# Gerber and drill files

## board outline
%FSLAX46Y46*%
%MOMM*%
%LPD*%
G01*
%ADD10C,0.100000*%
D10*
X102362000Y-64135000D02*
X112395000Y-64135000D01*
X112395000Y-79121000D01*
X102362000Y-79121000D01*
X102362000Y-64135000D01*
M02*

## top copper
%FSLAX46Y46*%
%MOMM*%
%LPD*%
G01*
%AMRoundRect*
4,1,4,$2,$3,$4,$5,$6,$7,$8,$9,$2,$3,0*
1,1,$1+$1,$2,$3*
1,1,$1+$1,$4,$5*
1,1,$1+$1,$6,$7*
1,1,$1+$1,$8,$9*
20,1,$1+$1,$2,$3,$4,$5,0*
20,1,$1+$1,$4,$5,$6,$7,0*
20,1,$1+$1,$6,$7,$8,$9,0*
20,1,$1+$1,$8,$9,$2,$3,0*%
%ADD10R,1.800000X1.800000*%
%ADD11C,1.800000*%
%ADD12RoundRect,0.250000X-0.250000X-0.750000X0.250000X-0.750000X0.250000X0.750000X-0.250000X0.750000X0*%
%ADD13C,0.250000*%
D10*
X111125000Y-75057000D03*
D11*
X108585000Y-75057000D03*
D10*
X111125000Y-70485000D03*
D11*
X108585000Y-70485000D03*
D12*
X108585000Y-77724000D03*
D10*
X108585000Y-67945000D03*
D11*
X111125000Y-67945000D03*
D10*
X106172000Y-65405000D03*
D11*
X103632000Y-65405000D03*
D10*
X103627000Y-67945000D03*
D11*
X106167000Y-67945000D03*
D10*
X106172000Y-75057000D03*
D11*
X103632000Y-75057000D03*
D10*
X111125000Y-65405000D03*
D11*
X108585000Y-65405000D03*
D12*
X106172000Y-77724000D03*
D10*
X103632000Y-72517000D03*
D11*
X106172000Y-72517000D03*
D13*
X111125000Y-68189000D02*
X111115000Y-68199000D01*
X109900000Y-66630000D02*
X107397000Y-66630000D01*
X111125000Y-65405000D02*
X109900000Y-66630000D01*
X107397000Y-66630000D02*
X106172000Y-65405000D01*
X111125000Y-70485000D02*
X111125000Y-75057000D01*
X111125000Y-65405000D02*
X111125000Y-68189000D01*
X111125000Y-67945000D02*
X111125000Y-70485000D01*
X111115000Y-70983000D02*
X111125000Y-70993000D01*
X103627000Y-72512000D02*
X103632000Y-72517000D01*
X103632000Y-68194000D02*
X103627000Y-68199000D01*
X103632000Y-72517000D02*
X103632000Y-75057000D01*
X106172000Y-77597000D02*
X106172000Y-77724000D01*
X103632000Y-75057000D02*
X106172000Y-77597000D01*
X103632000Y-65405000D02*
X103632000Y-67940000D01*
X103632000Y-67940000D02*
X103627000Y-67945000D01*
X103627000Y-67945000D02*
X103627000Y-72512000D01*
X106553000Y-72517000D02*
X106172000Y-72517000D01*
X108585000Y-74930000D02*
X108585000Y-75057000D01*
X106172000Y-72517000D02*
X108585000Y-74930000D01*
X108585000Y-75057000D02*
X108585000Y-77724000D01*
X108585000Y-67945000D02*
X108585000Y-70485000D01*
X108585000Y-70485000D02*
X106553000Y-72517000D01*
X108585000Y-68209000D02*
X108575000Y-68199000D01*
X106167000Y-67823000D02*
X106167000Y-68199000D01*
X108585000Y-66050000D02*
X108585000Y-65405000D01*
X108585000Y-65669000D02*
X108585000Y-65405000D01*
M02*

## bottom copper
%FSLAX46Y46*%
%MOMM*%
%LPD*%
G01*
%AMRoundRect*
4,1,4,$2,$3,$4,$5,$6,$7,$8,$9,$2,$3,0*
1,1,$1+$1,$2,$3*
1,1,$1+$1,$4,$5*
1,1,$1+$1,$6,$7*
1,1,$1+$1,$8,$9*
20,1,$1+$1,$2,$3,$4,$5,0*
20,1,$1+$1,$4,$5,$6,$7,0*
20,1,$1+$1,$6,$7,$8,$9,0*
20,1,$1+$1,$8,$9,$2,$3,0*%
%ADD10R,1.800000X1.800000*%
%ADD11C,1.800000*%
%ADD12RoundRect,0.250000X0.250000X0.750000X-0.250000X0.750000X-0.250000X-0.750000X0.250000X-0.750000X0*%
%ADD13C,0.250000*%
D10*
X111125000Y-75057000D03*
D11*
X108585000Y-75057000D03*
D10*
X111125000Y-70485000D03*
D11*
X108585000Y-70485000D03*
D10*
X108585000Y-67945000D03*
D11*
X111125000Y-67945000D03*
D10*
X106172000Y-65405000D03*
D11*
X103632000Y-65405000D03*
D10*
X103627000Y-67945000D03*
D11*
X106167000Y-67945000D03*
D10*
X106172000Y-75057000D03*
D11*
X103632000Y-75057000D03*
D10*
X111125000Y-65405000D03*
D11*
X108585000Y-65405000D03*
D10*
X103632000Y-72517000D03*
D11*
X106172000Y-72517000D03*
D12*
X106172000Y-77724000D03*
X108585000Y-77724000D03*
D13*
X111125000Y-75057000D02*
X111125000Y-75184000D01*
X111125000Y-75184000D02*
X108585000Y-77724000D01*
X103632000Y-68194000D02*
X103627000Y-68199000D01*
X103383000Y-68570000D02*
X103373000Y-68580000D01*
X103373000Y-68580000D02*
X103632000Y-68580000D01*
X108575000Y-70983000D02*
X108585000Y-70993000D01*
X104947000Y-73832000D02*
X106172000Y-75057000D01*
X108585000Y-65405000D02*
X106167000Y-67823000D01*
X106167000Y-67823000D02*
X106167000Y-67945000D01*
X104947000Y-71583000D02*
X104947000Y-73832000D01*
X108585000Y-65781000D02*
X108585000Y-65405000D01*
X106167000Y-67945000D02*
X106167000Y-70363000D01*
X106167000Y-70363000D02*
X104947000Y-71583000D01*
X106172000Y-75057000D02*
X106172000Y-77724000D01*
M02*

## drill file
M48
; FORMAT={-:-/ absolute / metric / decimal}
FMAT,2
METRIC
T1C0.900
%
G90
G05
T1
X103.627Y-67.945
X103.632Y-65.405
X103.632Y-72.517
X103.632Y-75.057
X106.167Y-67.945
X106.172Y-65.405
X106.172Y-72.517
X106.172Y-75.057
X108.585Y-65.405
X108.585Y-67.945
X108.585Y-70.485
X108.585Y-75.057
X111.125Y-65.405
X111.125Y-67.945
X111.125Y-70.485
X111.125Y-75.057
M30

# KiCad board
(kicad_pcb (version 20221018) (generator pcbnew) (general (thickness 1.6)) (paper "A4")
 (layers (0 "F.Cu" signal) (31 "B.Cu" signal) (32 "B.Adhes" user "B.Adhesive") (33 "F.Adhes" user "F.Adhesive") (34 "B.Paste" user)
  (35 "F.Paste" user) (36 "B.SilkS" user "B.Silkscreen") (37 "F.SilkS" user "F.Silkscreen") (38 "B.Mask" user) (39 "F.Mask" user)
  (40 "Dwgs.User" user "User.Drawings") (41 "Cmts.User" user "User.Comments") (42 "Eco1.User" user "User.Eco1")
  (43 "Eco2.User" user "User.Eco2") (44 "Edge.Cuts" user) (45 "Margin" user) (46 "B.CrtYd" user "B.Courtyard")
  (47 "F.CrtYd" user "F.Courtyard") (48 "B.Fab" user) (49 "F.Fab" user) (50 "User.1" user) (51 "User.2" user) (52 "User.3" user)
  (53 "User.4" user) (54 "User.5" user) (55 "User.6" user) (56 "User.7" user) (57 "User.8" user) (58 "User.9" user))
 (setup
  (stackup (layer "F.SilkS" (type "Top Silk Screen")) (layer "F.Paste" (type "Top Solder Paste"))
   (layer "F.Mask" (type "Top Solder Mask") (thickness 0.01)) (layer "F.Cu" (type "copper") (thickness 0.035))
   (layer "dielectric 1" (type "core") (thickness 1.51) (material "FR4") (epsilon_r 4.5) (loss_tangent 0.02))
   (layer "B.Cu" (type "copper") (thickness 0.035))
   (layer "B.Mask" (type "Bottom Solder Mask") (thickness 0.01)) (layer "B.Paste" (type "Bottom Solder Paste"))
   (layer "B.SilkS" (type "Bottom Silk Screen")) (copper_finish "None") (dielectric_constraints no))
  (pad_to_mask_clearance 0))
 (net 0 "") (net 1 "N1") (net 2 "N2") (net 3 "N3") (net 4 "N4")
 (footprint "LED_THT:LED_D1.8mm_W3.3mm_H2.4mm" (layer "F.Cu") (at 111.125 75.057 180)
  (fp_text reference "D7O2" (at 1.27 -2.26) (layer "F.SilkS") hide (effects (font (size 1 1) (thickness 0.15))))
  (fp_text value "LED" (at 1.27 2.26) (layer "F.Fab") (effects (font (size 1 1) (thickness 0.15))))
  (pad "1" thru_hole rect (at 0 0 180) (size 1.8 1.8) (drill 0.9) (layers "*.Cu" "*.Mask") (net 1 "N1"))
  (pad "2" thru_hole circle (at 2.54 0 180) (size 1.8 1.8) (drill 0.9) (layers "*.Cu" "*.Mask") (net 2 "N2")))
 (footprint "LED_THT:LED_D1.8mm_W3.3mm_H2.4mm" (layer "F.Cu") (at 111.125 70.485 180)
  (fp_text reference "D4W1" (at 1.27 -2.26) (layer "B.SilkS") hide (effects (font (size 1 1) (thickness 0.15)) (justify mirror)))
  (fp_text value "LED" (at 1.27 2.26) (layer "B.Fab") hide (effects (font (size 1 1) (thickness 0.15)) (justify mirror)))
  (pad "1" thru_hole rect (at 0 0 180) (size 1.8 1.8) (drill 0.9) (layers "*.Cu" "*.Mask") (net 1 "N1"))
  (pad "2" thru_hole circle (at 2.54 0 180) (size 1.8 1.8) (drill 0.9) (layers "*.Cu" "*.Mask") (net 2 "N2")))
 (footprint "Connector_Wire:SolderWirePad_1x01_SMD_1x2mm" (layer "F.Cu") (at 108.585 77.724)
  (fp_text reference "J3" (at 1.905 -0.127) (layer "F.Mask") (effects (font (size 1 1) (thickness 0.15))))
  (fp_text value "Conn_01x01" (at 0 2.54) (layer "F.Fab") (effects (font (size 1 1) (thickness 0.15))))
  (pad "1" smd roundrect (at 0 0) (size 1 2) (layers "F.Cu" "F.Paste" "F.Mask") (roundrect_rratio 0.25) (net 2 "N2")))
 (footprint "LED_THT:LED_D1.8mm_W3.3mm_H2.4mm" (layer "F.Cu") (at 108.585 67.945)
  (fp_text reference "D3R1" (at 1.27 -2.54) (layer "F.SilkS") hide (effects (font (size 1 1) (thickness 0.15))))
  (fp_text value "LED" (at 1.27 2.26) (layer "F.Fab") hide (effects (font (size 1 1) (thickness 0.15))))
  (pad "1" thru_hole rect (at 0 0) (size 1.8 1.8) (drill 0.9) (layers "*.Cu" "*.Mask") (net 2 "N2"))
  (pad "2" thru_hole circle (at 2.54 0) (size 1.8 1.8) (drill 0.9) (layers "*.Cu" "*.Mask") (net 1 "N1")))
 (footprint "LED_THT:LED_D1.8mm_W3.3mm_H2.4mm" (layer "F.Cu") (at 106.172 65.405 180)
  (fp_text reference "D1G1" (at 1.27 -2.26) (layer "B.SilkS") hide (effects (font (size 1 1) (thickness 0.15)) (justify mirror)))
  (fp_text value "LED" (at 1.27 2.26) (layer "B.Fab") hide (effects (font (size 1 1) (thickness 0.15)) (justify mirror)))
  (pad "1" thru_hole rect (at 0 0 180) (size 1.8 1.8) (drill 0.9) (layers "*.Cu" "*.Mask") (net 1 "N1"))
  (pad "2" thru_hole circle (at 2.54 0 180) (size 1.8 1.8) (drill 0.9) (layers "*.Cu" "*.Mask") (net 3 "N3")))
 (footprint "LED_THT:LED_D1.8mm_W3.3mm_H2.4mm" (layer "F.Cu") (at 103.627 67.945)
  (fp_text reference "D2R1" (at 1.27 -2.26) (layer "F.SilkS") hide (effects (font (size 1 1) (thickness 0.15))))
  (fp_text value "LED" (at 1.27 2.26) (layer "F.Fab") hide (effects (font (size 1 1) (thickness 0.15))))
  (pad "1" thru_hole rect (at 0 0) (size 1.8 1.8) (drill 0.9) (layers "*.Cu" "*.Mask") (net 3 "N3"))
  (pad "2" thru_hole circle (at 2.54 0) (size 1.8 1.8) (drill 0.9) (layers "*.Cu" "*.Mask") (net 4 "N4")))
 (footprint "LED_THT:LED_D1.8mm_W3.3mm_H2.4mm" (layer "F.Cu") (at 106.172 75.057 180)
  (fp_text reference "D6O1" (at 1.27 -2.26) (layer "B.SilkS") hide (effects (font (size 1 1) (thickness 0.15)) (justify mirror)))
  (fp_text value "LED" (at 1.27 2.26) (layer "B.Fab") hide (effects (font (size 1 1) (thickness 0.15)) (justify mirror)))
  (pad "1" thru_hole rect (at 0 0 180) (size 1.8 1.8) (drill 0.9) (layers "*.Cu" "*.Mask") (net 4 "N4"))
  (pad "2" thru_hole circle (at 2.54 0 180) (size 1.8 1.8) (drill 0.9) (layers "*.Cu" "*.Mask") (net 3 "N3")))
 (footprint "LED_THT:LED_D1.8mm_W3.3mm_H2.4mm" (layer "F.Cu") (at 111.125 65.405 180)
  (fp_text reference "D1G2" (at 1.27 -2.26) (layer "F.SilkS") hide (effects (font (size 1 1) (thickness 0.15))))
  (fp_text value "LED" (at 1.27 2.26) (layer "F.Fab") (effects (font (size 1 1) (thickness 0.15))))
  (pad "1" thru_hole rect (at 0 0 180) (size 1.8 1.8) (drill 0.9) (layers "*.Cu" "*.Mask") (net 1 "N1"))
  (pad "2" thru_hole circle (at 2.54 0 180) (size 1.8 1.8) (drill 0.9) (layers "*.Cu" "*.Mask") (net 4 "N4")))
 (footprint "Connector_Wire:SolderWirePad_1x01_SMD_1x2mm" (layer "F.Cu") (at 106.172 77.724)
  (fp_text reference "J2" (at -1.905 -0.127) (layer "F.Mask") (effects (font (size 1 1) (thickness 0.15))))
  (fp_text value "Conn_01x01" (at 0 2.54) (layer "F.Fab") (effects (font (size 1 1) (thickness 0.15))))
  (pad "1" smd roundrect (at 0 0) (size 1 2) (layers "F.Cu" "F.Paste" "F.Mask") (roundrect_rratio 0.25) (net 3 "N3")))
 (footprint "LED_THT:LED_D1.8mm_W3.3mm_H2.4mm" (layer "F.Cu") (at 103.632 72.517)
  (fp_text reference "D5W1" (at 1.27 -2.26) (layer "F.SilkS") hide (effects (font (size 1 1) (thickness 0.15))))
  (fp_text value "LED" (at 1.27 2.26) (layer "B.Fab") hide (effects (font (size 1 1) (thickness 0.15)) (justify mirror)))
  (pad "1" thru_hole rect (at 0 0) (size 1.8 1.8) (drill 0.9) (layers "*.Cu" "*.Mask") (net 3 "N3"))
  (pad "2" thru_hole circle (at 2.54 0) (size 1.8 1.8) (drill 0.9) (layers "*.Cu" "*.Mask") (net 2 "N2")))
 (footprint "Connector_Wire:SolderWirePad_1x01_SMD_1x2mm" (layer "B.Cu") (at 106.172 77.724 180)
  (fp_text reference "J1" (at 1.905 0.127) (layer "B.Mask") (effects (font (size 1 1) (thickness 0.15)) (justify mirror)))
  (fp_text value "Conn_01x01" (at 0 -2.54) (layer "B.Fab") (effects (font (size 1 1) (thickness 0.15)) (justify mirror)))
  (pad "1" smd roundrect (at 0 0 180) (size 1 2) (layers "B.Cu" "B.Paste" "B.Mask") (roundrect_rratio 0.25) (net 4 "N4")))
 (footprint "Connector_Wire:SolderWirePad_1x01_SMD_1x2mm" (layer "B.Cu") (at 108.585 77.724 180)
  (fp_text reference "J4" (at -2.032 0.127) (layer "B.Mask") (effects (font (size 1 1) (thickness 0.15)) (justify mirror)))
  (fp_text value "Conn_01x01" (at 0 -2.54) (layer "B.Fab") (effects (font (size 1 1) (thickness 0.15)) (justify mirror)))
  (pad "1" smd roundrect (at 0 0 180) (size 1 2) (layers "B.Cu" "B.Paste" "B.Mask") (roundrect_rratio 0.25) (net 1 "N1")))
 (gr_rect (start 102.362 64.135) (end 112.395 79.121) (stroke (width 0.1) (type default)) (fill none) (layer "Edge.Cuts"))
 (segment (start 111.125 68.189) (end 111.115 68.199) (width 0.25) (layer "F.Cu") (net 1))
 (segment (start 109.9 66.63) (end 107.397 66.63) (width 0.25) (layer "F.Cu") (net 1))
 (segment (start 111.125 65.405) (end 109.9 66.63) (width 0.25) (layer "F.Cu") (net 1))
 (segment (start 107.397 66.63) (end 106.172 65.405) (width 0.25) (layer "F.Cu") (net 1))
 (segment (start 111.125 70.485) (end 111.125 75.057) (width 0.25) (layer "F.Cu") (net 1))
 (segment (start 111.125 65.405) (end 111.125 68.189) (width 0.25) (layer "F.Cu") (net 1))
 (segment (start 111.125 67.945) (end 111.125 70.485) (width 0.25) (layer "F.Cu") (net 1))
 (segment (start 111.115 70.983) (end 111.125 70.993) (width 0.25) (layer "F.Cu") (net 1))
 (segment (start 111.125 75.057) (end 111.125 75.184) (width 0.25) (layer "B.Cu") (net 1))
 (segment (start 111.125 75.184) (end 108.585 77.724) (width 0.25) (layer "B.Cu") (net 1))
 (segment (start 103.627 72.512) (end 103.632 72.517) (width 0.25) (layer "F.Cu") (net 3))
 (segment (start 103.632 68.194) (end 103.627 68.199) (width 0.25) (layer "F.Cu") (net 3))
 (segment (start 103.632 72.517) (end 103.632 75.057) (width 0.25) (layer "F.Cu") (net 3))
 (segment (start 106.172 77.597) (end 106.172 77.724) (width 0.25) (layer "F.Cu") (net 3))
 (segment (start 103.632 75.057) (end 106.172 77.597) (width 0.25) (layer "F.Cu") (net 3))
 (segment (start 103.632 65.405) (end 103.632 67.94) (width 0.25) (layer "F.Cu") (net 3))
 (segment (start 103.632 67.94) (end 103.627 67.945) (width 0.25) (layer "F.Cu") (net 3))
 (segment (start 103.627 67.945) (end 103.627 72.512) (width 0.25) (layer "F.Cu") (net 3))
 (segment (start 103.632 68.194) (end 103.627 68.199) (width 0.25) (layer "B.Cu") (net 3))
 (segment (start 103.383 68.57) (end 103.373 68.58) (width 0.25) (layer "B.Cu") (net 3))
 (segment (start 103.373 68.58) (end 103.632 68.58) (width 0.25) (layer "B.Cu") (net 3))
 (segment (start 106.553 72.517) (end 106.172 72.517) (width 0.25) (layer "F.Cu") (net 2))
 (segment (start 108.585 74.93) (end 108.585 75.057) (width 0.25) (layer "F.Cu") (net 2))
 (segment (start 106.172 72.517) (end 108.585 74.93) (width 0.25) (layer "F.Cu") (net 2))
 (segment (start 108.585 75.057) (end 108.585 77.724) (width 0.25) (layer "F.Cu") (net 2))
 (segment (start 108.585 67.945) (end 108.585 70.485) (width 0.25) (layer "F.Cu") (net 2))
 (segment (start 108.585 70.485) (end 106.553 72.517) (width 0.25) (layer "F.Cu") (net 2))
 (segment (start 108.585 68.209) (end 108.575 68.199) (width 0.25) (layer "F.Cu") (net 2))
 (segment (start 108.575 70.983) (end 108.585 70.993) (width 0.25) (layer "B.Cu") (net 2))
 (segment (start 106.167 67.823) (end 106.167 68.199) (width 0.25) (layer "F.Cu") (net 4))
 (segment (start 108.585 66.05) (end 108.585 65.405) (width 0.25) (layer "F.Cu") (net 4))
 (segment (start 108.585 65.669) (end 108.585 65.405) (width 0.25) (layer "F.Cu") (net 4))
 (segment (start 104.947 73.832) (end 106.172 75.057) (width 0.25) (layer "B.Cu") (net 4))
 (segment (start 108.585 65.405) (end 106.167 67.823) (width 0.25) (layer "B.Cu") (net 4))
 (segment (start 106.167 67.823) (end 106.167 67.945) (width 0.25) (layer "B.Cu") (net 4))
 (segment (start 104.947 71.583) (end 104.947 73.832) (width 0.25) (layer "B.Cu") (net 4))
 (segment (start 108.585 65.781) (end 108.585 65.405) (width 0.25) (layer "B.Cu") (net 4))
 (segment (start 106.167 67.945) (end 106.167 70.363) (width 0.25) (layer "B.Cu") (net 4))
 (segment (start 106.167 70.363) (end 104.947 71.583) (width 0.25) (layer "B.Cu") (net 4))
 (segment (start 106.172 75.057) (end 106.172 77.724) (width 0.25) (layer "B.Cu") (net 4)))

